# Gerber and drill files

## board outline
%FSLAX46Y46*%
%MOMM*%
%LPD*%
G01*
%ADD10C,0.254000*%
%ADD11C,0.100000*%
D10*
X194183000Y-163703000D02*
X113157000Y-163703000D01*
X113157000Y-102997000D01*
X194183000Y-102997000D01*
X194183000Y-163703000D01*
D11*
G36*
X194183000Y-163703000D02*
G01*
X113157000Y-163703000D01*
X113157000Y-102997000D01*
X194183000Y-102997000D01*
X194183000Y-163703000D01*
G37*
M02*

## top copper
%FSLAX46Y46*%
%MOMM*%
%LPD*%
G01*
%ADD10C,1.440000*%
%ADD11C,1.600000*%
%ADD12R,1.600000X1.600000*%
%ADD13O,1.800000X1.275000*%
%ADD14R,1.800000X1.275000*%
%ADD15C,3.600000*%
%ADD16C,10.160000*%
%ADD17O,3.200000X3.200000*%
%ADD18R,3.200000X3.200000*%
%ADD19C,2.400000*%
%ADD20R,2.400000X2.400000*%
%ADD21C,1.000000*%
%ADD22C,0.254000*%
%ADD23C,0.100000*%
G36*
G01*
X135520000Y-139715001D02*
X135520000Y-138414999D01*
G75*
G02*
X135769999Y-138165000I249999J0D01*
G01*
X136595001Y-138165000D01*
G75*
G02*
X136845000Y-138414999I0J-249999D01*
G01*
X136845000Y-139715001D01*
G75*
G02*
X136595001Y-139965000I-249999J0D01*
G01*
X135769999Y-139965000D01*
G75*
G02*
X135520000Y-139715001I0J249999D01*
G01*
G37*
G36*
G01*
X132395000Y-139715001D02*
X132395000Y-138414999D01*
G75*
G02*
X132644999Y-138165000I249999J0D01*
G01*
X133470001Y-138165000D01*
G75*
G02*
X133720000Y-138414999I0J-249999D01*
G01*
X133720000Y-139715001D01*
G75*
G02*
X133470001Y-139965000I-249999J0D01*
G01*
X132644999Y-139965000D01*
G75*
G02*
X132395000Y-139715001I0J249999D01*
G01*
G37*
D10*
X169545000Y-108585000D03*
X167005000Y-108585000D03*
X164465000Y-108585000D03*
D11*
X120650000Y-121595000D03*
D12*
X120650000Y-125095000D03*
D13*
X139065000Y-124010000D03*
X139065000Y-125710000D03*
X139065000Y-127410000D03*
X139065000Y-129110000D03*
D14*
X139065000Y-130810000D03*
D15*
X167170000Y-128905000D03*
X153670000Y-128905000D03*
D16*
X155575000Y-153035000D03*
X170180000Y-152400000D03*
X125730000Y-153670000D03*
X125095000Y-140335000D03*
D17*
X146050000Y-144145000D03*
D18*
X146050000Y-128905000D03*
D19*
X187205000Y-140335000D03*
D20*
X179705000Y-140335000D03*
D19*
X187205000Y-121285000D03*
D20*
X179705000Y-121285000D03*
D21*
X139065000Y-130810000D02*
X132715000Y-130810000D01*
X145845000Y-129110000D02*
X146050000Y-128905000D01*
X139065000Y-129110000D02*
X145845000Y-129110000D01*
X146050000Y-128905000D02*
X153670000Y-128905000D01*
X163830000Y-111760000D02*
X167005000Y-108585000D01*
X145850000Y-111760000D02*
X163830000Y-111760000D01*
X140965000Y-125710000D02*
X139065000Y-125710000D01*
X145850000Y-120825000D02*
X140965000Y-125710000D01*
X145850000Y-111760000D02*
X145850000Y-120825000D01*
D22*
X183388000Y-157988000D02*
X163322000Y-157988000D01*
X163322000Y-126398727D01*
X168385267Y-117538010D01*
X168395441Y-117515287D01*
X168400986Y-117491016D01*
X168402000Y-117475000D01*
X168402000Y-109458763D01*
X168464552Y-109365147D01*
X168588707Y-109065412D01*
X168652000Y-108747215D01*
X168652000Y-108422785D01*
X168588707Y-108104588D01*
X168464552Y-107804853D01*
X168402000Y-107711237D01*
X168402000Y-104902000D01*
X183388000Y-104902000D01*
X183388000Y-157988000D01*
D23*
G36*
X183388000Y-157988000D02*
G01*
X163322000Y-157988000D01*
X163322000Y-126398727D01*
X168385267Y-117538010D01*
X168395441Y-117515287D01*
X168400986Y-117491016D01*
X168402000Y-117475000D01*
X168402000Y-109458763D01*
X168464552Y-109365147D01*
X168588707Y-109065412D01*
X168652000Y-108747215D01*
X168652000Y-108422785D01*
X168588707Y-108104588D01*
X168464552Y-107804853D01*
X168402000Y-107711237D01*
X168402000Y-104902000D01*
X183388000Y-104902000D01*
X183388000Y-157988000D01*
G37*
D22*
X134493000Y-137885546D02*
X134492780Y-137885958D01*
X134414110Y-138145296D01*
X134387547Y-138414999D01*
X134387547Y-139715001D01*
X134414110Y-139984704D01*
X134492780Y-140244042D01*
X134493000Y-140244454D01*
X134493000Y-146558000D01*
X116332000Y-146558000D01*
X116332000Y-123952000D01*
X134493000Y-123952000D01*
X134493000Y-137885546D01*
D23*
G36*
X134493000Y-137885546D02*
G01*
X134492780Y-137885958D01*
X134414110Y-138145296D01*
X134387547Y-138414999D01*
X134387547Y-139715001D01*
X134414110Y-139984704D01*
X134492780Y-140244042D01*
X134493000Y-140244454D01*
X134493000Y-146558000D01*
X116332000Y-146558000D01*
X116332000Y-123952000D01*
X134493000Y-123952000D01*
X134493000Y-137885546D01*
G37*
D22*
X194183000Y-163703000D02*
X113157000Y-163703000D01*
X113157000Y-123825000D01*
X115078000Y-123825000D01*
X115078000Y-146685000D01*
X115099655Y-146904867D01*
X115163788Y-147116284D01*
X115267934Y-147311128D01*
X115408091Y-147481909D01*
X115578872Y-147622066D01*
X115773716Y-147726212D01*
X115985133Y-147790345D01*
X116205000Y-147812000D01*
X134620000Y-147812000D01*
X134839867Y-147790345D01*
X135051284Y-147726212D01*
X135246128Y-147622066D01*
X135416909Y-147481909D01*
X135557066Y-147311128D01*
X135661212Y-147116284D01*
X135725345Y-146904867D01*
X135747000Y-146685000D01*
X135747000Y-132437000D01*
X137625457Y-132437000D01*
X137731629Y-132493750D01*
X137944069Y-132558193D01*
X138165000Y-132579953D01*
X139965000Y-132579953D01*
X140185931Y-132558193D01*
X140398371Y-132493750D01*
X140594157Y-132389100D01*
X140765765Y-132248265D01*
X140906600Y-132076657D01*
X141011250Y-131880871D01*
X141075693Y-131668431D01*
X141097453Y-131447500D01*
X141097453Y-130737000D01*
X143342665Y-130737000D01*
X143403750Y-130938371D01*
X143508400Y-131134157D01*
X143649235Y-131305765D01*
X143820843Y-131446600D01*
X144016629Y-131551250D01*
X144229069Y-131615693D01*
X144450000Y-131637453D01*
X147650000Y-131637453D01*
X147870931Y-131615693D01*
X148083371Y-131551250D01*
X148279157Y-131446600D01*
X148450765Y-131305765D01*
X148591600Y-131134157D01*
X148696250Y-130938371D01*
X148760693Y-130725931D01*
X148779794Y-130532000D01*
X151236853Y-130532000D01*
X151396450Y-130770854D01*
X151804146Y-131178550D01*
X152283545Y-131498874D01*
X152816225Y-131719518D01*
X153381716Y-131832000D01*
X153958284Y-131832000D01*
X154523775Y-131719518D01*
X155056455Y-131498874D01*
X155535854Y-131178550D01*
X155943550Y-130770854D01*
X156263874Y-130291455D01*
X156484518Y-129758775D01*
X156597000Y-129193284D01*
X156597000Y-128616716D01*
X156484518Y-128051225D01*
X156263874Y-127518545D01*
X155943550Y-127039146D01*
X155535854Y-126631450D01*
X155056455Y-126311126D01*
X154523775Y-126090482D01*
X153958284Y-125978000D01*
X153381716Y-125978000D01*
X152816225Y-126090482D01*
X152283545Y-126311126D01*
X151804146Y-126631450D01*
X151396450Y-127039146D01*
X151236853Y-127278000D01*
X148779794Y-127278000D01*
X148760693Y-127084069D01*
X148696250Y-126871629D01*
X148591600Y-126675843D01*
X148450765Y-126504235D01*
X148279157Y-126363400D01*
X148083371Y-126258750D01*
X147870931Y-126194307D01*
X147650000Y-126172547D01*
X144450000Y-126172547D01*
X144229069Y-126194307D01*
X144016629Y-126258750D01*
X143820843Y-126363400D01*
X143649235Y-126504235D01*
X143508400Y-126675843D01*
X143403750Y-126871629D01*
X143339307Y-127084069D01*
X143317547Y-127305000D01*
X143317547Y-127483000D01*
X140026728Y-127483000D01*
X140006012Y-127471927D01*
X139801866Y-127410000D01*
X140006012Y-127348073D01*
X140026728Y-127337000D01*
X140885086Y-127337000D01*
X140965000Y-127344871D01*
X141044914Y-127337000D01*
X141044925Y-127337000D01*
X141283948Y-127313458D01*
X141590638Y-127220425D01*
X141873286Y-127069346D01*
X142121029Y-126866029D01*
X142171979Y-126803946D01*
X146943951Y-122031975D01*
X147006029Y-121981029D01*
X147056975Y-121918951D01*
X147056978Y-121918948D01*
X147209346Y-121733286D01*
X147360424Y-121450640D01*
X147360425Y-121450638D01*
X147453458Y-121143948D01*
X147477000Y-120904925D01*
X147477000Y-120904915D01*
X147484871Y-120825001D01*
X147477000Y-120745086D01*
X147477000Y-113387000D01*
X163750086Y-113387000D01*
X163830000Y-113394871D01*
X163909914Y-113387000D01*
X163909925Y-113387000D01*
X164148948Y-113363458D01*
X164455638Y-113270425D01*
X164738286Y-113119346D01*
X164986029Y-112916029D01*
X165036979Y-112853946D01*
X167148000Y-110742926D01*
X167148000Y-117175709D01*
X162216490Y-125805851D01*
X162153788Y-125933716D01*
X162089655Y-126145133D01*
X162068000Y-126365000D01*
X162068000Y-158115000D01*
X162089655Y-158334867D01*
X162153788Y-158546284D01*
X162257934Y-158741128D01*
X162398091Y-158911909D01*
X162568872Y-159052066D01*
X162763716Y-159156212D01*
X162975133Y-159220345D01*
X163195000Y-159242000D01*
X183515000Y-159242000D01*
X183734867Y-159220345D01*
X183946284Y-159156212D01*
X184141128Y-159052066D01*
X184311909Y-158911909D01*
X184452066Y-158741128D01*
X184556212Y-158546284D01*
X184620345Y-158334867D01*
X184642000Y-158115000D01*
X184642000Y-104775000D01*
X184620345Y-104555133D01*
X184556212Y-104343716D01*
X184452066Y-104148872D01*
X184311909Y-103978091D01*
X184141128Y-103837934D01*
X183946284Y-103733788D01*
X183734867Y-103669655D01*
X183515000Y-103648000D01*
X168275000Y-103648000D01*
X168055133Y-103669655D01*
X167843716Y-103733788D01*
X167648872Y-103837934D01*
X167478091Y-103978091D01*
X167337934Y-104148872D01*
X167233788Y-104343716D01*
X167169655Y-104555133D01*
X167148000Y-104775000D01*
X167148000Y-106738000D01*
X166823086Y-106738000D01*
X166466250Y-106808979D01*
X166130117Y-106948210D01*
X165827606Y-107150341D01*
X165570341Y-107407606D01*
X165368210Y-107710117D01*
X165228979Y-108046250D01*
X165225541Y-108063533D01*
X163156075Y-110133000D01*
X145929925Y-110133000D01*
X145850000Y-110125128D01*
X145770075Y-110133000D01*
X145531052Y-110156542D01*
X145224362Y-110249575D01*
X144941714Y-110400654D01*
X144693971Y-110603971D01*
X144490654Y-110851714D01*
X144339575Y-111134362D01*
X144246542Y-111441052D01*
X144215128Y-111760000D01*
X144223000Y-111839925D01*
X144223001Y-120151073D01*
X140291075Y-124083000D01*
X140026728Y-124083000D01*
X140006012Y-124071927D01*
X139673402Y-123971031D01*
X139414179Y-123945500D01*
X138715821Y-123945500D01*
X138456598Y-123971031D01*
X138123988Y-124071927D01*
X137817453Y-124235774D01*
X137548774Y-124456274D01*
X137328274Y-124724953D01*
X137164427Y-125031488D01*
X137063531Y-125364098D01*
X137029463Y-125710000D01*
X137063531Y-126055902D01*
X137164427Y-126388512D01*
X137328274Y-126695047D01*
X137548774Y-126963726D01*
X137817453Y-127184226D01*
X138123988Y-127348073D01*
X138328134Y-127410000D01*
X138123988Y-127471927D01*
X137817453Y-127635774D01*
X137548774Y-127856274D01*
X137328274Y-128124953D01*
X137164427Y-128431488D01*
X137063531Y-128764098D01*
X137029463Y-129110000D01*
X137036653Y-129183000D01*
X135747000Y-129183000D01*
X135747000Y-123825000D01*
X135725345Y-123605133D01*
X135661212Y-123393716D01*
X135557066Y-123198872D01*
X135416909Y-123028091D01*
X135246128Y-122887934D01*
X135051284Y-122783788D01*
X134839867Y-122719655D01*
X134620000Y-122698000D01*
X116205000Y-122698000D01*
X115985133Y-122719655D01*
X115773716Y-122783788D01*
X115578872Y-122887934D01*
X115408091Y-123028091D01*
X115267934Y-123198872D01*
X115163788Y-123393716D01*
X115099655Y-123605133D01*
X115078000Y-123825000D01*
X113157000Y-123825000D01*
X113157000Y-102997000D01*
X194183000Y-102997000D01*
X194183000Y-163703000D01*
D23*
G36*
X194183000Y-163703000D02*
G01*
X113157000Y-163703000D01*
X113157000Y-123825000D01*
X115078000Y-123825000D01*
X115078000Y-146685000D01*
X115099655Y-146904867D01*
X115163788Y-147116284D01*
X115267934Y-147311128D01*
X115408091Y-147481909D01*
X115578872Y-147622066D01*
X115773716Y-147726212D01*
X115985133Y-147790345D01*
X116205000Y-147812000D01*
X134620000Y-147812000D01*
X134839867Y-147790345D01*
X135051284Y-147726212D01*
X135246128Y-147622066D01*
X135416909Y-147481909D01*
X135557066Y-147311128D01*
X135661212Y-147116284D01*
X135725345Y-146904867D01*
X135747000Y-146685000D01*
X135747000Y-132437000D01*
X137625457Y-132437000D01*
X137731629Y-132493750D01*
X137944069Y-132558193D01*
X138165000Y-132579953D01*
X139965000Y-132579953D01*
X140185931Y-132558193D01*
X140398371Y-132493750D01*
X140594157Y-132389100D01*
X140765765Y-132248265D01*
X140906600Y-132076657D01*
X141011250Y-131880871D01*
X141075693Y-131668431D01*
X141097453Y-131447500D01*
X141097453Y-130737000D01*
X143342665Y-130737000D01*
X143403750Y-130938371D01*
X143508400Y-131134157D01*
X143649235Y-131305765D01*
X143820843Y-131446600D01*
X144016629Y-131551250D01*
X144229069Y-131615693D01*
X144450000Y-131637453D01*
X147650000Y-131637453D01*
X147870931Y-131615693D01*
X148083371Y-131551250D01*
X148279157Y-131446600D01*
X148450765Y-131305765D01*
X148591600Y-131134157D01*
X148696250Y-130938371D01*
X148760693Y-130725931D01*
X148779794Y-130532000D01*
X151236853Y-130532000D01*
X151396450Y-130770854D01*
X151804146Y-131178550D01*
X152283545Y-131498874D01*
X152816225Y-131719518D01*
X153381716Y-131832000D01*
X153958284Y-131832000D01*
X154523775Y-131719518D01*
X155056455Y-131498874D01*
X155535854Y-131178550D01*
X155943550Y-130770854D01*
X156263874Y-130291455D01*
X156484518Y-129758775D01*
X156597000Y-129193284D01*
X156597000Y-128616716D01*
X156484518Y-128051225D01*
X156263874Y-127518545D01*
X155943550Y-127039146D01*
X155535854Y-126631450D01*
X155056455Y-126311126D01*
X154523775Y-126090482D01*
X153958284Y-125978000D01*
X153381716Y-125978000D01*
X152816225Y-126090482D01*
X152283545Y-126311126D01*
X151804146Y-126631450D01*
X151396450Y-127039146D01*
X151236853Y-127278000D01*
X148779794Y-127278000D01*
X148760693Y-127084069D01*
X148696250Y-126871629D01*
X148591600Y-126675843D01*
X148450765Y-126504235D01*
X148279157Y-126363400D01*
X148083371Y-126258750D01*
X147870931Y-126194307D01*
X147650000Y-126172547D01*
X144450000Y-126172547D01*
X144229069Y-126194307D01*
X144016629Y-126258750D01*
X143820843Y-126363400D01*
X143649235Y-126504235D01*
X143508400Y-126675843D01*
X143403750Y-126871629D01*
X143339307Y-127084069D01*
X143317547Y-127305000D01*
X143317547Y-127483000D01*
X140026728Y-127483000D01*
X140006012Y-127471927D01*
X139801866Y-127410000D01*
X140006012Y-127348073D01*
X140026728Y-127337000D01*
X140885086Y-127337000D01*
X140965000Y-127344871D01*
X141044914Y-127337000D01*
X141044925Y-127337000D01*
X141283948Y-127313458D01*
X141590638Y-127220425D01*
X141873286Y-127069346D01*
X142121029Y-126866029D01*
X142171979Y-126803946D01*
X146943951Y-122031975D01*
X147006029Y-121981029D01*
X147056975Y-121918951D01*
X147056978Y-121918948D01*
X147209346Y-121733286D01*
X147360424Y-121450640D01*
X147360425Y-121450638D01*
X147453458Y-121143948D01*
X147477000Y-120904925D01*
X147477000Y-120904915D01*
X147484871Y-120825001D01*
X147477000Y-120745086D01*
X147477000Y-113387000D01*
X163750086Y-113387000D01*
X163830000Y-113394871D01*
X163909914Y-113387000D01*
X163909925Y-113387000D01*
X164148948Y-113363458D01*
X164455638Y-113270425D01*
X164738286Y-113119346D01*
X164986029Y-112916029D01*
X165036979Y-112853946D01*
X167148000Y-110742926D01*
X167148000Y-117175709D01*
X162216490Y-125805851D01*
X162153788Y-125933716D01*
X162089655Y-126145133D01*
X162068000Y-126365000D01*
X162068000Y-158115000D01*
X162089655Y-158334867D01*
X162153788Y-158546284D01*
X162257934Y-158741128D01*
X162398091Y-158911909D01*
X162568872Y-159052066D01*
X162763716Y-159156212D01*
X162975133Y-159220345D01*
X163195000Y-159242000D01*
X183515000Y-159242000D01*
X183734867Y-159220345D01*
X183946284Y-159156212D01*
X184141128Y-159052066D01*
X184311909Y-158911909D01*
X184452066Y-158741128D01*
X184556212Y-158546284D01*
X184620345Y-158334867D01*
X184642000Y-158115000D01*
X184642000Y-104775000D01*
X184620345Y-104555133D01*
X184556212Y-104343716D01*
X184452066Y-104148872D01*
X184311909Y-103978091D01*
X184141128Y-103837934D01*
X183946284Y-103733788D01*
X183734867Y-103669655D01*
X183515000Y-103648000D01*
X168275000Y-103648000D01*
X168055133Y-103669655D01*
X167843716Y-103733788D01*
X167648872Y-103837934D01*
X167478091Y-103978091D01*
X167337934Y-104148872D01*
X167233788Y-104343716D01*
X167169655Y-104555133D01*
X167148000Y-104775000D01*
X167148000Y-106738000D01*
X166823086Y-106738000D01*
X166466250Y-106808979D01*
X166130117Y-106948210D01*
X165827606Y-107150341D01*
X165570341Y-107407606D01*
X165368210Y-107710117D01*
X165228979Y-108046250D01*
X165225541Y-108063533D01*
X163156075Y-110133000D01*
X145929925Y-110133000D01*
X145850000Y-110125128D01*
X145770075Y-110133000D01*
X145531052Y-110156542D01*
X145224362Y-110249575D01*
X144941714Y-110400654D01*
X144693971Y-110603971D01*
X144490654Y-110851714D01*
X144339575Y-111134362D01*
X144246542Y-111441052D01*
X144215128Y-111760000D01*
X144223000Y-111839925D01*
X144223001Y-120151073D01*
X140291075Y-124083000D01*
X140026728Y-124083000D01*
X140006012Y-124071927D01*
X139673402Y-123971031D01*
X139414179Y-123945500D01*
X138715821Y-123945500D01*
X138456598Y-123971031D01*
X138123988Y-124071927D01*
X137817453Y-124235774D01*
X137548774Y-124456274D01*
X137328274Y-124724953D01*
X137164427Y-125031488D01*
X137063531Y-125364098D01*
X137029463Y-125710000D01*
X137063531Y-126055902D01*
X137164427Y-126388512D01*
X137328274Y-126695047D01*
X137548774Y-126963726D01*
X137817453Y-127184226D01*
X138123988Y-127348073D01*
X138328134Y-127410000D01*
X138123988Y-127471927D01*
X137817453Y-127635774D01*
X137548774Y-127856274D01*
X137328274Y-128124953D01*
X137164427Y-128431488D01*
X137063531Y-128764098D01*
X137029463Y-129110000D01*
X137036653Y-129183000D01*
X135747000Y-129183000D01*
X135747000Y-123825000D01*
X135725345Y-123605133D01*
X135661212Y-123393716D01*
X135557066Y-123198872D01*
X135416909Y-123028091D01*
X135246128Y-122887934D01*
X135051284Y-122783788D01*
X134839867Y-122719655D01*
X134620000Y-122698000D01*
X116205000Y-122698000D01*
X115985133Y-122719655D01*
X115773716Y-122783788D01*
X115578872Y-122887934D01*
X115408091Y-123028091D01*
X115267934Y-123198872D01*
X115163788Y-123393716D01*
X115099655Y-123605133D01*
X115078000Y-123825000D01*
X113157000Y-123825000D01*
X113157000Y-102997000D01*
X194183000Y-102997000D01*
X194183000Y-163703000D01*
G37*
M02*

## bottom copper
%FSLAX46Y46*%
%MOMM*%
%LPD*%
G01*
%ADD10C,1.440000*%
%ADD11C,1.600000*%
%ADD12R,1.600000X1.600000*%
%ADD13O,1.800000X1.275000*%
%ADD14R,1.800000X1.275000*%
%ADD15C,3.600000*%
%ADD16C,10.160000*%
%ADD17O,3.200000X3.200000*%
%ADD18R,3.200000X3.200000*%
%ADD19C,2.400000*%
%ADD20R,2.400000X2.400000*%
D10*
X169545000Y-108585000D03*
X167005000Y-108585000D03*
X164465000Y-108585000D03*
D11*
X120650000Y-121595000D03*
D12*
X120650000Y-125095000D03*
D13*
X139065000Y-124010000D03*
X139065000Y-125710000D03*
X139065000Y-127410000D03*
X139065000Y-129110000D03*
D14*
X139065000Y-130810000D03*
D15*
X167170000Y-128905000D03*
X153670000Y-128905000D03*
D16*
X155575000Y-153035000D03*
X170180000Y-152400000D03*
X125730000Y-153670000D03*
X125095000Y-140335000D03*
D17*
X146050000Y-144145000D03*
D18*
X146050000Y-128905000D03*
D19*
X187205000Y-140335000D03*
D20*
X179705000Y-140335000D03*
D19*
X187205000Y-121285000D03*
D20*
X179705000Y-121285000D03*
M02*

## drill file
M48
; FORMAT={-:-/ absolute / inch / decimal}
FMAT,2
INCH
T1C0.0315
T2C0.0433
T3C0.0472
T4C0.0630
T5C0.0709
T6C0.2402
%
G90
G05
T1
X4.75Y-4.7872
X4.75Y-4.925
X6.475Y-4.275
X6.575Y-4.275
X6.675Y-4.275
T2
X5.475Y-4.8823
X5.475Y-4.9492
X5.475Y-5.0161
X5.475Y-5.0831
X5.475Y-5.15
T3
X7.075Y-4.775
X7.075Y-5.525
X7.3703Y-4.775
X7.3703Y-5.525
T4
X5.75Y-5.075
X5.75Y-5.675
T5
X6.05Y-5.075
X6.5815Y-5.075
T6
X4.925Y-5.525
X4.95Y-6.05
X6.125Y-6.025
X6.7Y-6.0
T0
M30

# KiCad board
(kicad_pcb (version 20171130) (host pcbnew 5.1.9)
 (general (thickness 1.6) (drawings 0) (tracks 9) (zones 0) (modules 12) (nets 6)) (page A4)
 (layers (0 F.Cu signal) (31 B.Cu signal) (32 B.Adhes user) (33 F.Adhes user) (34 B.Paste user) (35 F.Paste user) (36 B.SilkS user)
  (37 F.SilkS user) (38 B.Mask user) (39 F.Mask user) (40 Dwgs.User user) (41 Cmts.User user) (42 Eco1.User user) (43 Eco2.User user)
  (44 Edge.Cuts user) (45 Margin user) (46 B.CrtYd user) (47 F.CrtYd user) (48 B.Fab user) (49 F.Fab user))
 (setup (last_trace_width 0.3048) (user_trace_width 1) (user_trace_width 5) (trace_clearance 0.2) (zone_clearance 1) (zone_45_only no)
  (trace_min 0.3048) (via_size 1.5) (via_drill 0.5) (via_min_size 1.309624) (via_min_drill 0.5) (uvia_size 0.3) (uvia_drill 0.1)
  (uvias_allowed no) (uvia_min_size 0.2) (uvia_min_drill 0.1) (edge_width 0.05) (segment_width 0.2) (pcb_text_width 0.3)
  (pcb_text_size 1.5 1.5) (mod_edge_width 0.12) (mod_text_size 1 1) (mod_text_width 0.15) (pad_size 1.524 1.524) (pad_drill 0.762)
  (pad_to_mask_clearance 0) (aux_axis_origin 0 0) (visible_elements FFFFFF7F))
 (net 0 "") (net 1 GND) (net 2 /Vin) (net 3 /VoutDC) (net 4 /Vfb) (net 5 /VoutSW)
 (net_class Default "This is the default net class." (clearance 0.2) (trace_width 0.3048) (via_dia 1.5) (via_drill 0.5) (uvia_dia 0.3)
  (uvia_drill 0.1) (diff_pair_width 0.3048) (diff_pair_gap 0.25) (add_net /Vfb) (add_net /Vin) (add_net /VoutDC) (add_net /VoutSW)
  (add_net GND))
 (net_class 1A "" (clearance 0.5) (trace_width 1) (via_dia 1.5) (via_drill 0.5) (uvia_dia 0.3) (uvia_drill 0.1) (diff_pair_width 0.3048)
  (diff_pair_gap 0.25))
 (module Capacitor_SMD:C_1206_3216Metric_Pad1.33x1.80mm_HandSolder (layer F.Cu) (at 134.62 139.065)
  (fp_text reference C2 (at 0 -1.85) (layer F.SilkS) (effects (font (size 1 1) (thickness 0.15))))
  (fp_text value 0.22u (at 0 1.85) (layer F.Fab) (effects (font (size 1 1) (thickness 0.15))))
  (pad 2 smd roundrect (at 1.5625 0) (size 1.325 1.8) (layers F.Cu F.Paste F.Mask) (roundrect_rratio 0.1886784905660377) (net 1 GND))
  (pad 1 smd roundrect (at -1.5625 0) (size 1.325 1.8) (layers F.Cu F.Paste F.Mask) (roundrect_rratio 0.1886784905660377) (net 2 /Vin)))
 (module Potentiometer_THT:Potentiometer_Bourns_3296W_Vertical (layer F.Cu) (at 164.465 108.585 180)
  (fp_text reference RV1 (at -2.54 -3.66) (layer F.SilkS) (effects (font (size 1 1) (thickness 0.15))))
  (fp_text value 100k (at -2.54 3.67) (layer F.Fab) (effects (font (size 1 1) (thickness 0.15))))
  (pad 3 thru_hole circle (at -5.08 0 180) (size 1.44 1.44) (drill 0.8) (layers *.Cu *.Mask) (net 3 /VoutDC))
  (pad 2 thru_hole circle (at -2.54 0 180) (size 1.44 1.44) (drill 0.8) (layers *.Cu *.Mask) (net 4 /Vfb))
  (pad 1 thru_hole circle (at 0 0 180) (size 1.44 1.44) (drill 0.8) (layers *.Cu *.Mask) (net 1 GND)))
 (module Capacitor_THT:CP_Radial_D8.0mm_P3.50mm (layer F.Cu) (at 120.65 125.095 90)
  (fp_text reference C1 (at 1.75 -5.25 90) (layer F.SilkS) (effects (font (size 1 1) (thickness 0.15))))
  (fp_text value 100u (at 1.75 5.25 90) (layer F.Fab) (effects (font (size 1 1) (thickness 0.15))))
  (pad 2 thru_hole circle (at 3.5 0 90) (size 1.6 1.6) (drill 0.8) (layers *.Cu *.Mask) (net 1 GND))
  (pad 1 thru_hole rect (at 0 0 90) (size 1.6 1.6) (drill 0.8) (layers *.Cu *.Mask) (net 2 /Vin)))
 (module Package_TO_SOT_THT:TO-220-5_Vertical (layer F.Cu) (at 139.065 130.81 90)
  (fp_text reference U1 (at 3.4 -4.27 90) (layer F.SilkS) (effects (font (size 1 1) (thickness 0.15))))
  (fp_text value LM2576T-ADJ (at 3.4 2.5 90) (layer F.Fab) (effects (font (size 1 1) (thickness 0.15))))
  (pad 5 thru_hole oval (at 6.8 0 90) (size 1.275 1.8) (drill 1.1) (layers *.Cu *.Mask) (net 1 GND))
  (pad 4 thru_hole oval (at 5.1 0 90) (size 1.275 1.8) (drill 1.1) (layers *.Cu *.Mask) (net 4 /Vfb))
  (pad 3 thru_hole oval (at 3.4 0 90) (size 1.275 1.8) (drill 1.1) (layers *.Cu *.Mask) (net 1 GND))
  (pad 2 thru_hole oval (at 1.7 0 90) (size 1.275 1.8) (drill 1.1) (layers *.Cu *.Mask) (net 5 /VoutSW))
  (pad 1 thru_hole rect (at 0 0 90) (size 1.275 1.8) (drill 1.1) (layers *.Cu *.Mask) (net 2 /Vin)))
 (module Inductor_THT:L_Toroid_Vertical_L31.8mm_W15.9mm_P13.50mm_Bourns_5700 (layer F.Cu) (at 153.67 128.905 90)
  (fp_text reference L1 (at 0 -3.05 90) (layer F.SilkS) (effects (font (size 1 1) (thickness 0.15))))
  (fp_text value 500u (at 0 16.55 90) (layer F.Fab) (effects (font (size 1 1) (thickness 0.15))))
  (pad 2 thru_hole circle (at 0 13.5 90) (size 3.6 3.6) (drill 1.8) (layers *.Cu *.Mask) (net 3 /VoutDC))
  (pad 1 thru_hole circle (at 0 0 90) (size 3.6 3.6) (drill 1.8) (layers *.Cu *.Mask) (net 5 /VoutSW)))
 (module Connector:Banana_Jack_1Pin (layer F.Cu) (at 155.575 153.035)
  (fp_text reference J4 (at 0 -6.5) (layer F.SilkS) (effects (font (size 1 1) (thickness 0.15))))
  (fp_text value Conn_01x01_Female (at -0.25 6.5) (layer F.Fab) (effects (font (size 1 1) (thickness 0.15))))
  (pad 1 thru_hole circle (at 0 0) (size 10.16 10.16) (drill 6.1) (layers *.Cu *.Mask) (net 1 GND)))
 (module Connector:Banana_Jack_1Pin (layer F.Cu) (at 170.18 152.4)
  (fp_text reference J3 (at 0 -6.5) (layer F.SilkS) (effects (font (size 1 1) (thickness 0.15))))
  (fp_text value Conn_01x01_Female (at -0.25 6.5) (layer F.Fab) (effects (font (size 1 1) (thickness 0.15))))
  (pad 1 thru_hole circle (at 0 0) (size 10.16 10.16) (drill 6.1) (layers *.Cu *.Mask) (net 3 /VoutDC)))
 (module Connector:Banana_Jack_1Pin (layer F.Cu) (at 125.73 153.67)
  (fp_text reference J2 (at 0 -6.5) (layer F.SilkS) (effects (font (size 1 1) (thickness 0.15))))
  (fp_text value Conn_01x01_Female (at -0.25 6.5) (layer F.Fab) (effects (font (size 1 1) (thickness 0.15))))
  (pad 1 thru_hole circle (at 0 0) (size 10.16 10.16) (drill 6.1) (layers *.Cu *.Mask) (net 1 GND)))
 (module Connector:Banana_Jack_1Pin (layer F.Cu) (at 125.095 140.335)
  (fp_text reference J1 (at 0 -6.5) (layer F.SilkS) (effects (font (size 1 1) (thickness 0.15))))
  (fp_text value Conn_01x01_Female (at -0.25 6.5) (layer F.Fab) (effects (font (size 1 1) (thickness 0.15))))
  (pad 1 thru_hole circle (at 0 0) (size 10.16 10.16) (drill 6.1) (layers *.Cu *.Mask) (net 2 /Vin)))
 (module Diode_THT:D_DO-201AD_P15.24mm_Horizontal (layer F.Cu) (at 146.05 128.905 270)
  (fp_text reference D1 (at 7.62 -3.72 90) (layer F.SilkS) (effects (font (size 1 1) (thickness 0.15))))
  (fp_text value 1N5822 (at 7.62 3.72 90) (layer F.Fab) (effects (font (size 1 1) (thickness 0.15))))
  (pad 2 thru_hole oval (at 15.24 0 270) (size 3.2 3.2) (drill 1.6) (layers *.Cu *.Mask) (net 1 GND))
  (pad 1 thru_hole rect (at 0 0 270) (size 3.2 3.2) (drill 1.6) (layers *.Cu *.Mask) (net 5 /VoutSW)))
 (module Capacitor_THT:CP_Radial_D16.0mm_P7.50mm (layer F.Cu) (at 179.705 140.335)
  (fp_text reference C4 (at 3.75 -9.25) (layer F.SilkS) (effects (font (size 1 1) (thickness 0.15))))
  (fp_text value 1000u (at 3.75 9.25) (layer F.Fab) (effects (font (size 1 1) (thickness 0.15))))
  (pad 2 thru_hole circle (at 7.5 0) (size 2.4 2.4) (drill 1.2) (layers *.Cu *.Mask) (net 1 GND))
  (pad 1 thru_hole rect (at 0 0) (size 2.4 2.4) (drill 1.2) (layers *.Cu *.Mask) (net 3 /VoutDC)))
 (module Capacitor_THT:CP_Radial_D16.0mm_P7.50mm (layer F.Cu) (at 179.705 121.285)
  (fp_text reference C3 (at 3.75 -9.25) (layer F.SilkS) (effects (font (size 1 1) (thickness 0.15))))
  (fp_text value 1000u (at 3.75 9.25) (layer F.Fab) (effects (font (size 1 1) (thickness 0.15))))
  (pad 2 thru_hole circle (at 7.5 0) (size 2.4 2.4) (drill 1.2) (layers *.Cu *.Mask) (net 1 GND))
  (pad 1 thru_hole rect (at 0 0) (size 2.4 2.4) (drill 1.2) (layers *.Cu *.Mask) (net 3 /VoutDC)))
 (segment (start 139.065 130.81) (end 132.715 130.81) (width 1) (layer F.Cu) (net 2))
 (segment (start 145.845 129.11) (end 146.05 128.905) (width 1) (layer F.Cu) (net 5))
 (segment (start 139.065 129.11) (end 145.845 129.11) (width 1) (layer F.Cu) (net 5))
 (segment (start 146.05 128.905) (end 153.67 128.905) (width 1) (layer F.Cu) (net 5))
 (segment (start 163.83 111.76) (end 167.005 108.585) (width 1) (layer F.Cu) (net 4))
 (segment (start 145.85 111.76) (end 163.83 111.76) (width 1) (layer F.Cu) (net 4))
 (segment (start 140.965 125.71) (end 139.065 125.71) (width 1) (layer F.Cu) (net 4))
 (segment (start 145.85 120.825) (end 140.965 125.71) (width 1) (layer F.Cu) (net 4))
 (segment (start 145.85 111.76) (end 145.85 120.825) (width 1) (layer F.Cu) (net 4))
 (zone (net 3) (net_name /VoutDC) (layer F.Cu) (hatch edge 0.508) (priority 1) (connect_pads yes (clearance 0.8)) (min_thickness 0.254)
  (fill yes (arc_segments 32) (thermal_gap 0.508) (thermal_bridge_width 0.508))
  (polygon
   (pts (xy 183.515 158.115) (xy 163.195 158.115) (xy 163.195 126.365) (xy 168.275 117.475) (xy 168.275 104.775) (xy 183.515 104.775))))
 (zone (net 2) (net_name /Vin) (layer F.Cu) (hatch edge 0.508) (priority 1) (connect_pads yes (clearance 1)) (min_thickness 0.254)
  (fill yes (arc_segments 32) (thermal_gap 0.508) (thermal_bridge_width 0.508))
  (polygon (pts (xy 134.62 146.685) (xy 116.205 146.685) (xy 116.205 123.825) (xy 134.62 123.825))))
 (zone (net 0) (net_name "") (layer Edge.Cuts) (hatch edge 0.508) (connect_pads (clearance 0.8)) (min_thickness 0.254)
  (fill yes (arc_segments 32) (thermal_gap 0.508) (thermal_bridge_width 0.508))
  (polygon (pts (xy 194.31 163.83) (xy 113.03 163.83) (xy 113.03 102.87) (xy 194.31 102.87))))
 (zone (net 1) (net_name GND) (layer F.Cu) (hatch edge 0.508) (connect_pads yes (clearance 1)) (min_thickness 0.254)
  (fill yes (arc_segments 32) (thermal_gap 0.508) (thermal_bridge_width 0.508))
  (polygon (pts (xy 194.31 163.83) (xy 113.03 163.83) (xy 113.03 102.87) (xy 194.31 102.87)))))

